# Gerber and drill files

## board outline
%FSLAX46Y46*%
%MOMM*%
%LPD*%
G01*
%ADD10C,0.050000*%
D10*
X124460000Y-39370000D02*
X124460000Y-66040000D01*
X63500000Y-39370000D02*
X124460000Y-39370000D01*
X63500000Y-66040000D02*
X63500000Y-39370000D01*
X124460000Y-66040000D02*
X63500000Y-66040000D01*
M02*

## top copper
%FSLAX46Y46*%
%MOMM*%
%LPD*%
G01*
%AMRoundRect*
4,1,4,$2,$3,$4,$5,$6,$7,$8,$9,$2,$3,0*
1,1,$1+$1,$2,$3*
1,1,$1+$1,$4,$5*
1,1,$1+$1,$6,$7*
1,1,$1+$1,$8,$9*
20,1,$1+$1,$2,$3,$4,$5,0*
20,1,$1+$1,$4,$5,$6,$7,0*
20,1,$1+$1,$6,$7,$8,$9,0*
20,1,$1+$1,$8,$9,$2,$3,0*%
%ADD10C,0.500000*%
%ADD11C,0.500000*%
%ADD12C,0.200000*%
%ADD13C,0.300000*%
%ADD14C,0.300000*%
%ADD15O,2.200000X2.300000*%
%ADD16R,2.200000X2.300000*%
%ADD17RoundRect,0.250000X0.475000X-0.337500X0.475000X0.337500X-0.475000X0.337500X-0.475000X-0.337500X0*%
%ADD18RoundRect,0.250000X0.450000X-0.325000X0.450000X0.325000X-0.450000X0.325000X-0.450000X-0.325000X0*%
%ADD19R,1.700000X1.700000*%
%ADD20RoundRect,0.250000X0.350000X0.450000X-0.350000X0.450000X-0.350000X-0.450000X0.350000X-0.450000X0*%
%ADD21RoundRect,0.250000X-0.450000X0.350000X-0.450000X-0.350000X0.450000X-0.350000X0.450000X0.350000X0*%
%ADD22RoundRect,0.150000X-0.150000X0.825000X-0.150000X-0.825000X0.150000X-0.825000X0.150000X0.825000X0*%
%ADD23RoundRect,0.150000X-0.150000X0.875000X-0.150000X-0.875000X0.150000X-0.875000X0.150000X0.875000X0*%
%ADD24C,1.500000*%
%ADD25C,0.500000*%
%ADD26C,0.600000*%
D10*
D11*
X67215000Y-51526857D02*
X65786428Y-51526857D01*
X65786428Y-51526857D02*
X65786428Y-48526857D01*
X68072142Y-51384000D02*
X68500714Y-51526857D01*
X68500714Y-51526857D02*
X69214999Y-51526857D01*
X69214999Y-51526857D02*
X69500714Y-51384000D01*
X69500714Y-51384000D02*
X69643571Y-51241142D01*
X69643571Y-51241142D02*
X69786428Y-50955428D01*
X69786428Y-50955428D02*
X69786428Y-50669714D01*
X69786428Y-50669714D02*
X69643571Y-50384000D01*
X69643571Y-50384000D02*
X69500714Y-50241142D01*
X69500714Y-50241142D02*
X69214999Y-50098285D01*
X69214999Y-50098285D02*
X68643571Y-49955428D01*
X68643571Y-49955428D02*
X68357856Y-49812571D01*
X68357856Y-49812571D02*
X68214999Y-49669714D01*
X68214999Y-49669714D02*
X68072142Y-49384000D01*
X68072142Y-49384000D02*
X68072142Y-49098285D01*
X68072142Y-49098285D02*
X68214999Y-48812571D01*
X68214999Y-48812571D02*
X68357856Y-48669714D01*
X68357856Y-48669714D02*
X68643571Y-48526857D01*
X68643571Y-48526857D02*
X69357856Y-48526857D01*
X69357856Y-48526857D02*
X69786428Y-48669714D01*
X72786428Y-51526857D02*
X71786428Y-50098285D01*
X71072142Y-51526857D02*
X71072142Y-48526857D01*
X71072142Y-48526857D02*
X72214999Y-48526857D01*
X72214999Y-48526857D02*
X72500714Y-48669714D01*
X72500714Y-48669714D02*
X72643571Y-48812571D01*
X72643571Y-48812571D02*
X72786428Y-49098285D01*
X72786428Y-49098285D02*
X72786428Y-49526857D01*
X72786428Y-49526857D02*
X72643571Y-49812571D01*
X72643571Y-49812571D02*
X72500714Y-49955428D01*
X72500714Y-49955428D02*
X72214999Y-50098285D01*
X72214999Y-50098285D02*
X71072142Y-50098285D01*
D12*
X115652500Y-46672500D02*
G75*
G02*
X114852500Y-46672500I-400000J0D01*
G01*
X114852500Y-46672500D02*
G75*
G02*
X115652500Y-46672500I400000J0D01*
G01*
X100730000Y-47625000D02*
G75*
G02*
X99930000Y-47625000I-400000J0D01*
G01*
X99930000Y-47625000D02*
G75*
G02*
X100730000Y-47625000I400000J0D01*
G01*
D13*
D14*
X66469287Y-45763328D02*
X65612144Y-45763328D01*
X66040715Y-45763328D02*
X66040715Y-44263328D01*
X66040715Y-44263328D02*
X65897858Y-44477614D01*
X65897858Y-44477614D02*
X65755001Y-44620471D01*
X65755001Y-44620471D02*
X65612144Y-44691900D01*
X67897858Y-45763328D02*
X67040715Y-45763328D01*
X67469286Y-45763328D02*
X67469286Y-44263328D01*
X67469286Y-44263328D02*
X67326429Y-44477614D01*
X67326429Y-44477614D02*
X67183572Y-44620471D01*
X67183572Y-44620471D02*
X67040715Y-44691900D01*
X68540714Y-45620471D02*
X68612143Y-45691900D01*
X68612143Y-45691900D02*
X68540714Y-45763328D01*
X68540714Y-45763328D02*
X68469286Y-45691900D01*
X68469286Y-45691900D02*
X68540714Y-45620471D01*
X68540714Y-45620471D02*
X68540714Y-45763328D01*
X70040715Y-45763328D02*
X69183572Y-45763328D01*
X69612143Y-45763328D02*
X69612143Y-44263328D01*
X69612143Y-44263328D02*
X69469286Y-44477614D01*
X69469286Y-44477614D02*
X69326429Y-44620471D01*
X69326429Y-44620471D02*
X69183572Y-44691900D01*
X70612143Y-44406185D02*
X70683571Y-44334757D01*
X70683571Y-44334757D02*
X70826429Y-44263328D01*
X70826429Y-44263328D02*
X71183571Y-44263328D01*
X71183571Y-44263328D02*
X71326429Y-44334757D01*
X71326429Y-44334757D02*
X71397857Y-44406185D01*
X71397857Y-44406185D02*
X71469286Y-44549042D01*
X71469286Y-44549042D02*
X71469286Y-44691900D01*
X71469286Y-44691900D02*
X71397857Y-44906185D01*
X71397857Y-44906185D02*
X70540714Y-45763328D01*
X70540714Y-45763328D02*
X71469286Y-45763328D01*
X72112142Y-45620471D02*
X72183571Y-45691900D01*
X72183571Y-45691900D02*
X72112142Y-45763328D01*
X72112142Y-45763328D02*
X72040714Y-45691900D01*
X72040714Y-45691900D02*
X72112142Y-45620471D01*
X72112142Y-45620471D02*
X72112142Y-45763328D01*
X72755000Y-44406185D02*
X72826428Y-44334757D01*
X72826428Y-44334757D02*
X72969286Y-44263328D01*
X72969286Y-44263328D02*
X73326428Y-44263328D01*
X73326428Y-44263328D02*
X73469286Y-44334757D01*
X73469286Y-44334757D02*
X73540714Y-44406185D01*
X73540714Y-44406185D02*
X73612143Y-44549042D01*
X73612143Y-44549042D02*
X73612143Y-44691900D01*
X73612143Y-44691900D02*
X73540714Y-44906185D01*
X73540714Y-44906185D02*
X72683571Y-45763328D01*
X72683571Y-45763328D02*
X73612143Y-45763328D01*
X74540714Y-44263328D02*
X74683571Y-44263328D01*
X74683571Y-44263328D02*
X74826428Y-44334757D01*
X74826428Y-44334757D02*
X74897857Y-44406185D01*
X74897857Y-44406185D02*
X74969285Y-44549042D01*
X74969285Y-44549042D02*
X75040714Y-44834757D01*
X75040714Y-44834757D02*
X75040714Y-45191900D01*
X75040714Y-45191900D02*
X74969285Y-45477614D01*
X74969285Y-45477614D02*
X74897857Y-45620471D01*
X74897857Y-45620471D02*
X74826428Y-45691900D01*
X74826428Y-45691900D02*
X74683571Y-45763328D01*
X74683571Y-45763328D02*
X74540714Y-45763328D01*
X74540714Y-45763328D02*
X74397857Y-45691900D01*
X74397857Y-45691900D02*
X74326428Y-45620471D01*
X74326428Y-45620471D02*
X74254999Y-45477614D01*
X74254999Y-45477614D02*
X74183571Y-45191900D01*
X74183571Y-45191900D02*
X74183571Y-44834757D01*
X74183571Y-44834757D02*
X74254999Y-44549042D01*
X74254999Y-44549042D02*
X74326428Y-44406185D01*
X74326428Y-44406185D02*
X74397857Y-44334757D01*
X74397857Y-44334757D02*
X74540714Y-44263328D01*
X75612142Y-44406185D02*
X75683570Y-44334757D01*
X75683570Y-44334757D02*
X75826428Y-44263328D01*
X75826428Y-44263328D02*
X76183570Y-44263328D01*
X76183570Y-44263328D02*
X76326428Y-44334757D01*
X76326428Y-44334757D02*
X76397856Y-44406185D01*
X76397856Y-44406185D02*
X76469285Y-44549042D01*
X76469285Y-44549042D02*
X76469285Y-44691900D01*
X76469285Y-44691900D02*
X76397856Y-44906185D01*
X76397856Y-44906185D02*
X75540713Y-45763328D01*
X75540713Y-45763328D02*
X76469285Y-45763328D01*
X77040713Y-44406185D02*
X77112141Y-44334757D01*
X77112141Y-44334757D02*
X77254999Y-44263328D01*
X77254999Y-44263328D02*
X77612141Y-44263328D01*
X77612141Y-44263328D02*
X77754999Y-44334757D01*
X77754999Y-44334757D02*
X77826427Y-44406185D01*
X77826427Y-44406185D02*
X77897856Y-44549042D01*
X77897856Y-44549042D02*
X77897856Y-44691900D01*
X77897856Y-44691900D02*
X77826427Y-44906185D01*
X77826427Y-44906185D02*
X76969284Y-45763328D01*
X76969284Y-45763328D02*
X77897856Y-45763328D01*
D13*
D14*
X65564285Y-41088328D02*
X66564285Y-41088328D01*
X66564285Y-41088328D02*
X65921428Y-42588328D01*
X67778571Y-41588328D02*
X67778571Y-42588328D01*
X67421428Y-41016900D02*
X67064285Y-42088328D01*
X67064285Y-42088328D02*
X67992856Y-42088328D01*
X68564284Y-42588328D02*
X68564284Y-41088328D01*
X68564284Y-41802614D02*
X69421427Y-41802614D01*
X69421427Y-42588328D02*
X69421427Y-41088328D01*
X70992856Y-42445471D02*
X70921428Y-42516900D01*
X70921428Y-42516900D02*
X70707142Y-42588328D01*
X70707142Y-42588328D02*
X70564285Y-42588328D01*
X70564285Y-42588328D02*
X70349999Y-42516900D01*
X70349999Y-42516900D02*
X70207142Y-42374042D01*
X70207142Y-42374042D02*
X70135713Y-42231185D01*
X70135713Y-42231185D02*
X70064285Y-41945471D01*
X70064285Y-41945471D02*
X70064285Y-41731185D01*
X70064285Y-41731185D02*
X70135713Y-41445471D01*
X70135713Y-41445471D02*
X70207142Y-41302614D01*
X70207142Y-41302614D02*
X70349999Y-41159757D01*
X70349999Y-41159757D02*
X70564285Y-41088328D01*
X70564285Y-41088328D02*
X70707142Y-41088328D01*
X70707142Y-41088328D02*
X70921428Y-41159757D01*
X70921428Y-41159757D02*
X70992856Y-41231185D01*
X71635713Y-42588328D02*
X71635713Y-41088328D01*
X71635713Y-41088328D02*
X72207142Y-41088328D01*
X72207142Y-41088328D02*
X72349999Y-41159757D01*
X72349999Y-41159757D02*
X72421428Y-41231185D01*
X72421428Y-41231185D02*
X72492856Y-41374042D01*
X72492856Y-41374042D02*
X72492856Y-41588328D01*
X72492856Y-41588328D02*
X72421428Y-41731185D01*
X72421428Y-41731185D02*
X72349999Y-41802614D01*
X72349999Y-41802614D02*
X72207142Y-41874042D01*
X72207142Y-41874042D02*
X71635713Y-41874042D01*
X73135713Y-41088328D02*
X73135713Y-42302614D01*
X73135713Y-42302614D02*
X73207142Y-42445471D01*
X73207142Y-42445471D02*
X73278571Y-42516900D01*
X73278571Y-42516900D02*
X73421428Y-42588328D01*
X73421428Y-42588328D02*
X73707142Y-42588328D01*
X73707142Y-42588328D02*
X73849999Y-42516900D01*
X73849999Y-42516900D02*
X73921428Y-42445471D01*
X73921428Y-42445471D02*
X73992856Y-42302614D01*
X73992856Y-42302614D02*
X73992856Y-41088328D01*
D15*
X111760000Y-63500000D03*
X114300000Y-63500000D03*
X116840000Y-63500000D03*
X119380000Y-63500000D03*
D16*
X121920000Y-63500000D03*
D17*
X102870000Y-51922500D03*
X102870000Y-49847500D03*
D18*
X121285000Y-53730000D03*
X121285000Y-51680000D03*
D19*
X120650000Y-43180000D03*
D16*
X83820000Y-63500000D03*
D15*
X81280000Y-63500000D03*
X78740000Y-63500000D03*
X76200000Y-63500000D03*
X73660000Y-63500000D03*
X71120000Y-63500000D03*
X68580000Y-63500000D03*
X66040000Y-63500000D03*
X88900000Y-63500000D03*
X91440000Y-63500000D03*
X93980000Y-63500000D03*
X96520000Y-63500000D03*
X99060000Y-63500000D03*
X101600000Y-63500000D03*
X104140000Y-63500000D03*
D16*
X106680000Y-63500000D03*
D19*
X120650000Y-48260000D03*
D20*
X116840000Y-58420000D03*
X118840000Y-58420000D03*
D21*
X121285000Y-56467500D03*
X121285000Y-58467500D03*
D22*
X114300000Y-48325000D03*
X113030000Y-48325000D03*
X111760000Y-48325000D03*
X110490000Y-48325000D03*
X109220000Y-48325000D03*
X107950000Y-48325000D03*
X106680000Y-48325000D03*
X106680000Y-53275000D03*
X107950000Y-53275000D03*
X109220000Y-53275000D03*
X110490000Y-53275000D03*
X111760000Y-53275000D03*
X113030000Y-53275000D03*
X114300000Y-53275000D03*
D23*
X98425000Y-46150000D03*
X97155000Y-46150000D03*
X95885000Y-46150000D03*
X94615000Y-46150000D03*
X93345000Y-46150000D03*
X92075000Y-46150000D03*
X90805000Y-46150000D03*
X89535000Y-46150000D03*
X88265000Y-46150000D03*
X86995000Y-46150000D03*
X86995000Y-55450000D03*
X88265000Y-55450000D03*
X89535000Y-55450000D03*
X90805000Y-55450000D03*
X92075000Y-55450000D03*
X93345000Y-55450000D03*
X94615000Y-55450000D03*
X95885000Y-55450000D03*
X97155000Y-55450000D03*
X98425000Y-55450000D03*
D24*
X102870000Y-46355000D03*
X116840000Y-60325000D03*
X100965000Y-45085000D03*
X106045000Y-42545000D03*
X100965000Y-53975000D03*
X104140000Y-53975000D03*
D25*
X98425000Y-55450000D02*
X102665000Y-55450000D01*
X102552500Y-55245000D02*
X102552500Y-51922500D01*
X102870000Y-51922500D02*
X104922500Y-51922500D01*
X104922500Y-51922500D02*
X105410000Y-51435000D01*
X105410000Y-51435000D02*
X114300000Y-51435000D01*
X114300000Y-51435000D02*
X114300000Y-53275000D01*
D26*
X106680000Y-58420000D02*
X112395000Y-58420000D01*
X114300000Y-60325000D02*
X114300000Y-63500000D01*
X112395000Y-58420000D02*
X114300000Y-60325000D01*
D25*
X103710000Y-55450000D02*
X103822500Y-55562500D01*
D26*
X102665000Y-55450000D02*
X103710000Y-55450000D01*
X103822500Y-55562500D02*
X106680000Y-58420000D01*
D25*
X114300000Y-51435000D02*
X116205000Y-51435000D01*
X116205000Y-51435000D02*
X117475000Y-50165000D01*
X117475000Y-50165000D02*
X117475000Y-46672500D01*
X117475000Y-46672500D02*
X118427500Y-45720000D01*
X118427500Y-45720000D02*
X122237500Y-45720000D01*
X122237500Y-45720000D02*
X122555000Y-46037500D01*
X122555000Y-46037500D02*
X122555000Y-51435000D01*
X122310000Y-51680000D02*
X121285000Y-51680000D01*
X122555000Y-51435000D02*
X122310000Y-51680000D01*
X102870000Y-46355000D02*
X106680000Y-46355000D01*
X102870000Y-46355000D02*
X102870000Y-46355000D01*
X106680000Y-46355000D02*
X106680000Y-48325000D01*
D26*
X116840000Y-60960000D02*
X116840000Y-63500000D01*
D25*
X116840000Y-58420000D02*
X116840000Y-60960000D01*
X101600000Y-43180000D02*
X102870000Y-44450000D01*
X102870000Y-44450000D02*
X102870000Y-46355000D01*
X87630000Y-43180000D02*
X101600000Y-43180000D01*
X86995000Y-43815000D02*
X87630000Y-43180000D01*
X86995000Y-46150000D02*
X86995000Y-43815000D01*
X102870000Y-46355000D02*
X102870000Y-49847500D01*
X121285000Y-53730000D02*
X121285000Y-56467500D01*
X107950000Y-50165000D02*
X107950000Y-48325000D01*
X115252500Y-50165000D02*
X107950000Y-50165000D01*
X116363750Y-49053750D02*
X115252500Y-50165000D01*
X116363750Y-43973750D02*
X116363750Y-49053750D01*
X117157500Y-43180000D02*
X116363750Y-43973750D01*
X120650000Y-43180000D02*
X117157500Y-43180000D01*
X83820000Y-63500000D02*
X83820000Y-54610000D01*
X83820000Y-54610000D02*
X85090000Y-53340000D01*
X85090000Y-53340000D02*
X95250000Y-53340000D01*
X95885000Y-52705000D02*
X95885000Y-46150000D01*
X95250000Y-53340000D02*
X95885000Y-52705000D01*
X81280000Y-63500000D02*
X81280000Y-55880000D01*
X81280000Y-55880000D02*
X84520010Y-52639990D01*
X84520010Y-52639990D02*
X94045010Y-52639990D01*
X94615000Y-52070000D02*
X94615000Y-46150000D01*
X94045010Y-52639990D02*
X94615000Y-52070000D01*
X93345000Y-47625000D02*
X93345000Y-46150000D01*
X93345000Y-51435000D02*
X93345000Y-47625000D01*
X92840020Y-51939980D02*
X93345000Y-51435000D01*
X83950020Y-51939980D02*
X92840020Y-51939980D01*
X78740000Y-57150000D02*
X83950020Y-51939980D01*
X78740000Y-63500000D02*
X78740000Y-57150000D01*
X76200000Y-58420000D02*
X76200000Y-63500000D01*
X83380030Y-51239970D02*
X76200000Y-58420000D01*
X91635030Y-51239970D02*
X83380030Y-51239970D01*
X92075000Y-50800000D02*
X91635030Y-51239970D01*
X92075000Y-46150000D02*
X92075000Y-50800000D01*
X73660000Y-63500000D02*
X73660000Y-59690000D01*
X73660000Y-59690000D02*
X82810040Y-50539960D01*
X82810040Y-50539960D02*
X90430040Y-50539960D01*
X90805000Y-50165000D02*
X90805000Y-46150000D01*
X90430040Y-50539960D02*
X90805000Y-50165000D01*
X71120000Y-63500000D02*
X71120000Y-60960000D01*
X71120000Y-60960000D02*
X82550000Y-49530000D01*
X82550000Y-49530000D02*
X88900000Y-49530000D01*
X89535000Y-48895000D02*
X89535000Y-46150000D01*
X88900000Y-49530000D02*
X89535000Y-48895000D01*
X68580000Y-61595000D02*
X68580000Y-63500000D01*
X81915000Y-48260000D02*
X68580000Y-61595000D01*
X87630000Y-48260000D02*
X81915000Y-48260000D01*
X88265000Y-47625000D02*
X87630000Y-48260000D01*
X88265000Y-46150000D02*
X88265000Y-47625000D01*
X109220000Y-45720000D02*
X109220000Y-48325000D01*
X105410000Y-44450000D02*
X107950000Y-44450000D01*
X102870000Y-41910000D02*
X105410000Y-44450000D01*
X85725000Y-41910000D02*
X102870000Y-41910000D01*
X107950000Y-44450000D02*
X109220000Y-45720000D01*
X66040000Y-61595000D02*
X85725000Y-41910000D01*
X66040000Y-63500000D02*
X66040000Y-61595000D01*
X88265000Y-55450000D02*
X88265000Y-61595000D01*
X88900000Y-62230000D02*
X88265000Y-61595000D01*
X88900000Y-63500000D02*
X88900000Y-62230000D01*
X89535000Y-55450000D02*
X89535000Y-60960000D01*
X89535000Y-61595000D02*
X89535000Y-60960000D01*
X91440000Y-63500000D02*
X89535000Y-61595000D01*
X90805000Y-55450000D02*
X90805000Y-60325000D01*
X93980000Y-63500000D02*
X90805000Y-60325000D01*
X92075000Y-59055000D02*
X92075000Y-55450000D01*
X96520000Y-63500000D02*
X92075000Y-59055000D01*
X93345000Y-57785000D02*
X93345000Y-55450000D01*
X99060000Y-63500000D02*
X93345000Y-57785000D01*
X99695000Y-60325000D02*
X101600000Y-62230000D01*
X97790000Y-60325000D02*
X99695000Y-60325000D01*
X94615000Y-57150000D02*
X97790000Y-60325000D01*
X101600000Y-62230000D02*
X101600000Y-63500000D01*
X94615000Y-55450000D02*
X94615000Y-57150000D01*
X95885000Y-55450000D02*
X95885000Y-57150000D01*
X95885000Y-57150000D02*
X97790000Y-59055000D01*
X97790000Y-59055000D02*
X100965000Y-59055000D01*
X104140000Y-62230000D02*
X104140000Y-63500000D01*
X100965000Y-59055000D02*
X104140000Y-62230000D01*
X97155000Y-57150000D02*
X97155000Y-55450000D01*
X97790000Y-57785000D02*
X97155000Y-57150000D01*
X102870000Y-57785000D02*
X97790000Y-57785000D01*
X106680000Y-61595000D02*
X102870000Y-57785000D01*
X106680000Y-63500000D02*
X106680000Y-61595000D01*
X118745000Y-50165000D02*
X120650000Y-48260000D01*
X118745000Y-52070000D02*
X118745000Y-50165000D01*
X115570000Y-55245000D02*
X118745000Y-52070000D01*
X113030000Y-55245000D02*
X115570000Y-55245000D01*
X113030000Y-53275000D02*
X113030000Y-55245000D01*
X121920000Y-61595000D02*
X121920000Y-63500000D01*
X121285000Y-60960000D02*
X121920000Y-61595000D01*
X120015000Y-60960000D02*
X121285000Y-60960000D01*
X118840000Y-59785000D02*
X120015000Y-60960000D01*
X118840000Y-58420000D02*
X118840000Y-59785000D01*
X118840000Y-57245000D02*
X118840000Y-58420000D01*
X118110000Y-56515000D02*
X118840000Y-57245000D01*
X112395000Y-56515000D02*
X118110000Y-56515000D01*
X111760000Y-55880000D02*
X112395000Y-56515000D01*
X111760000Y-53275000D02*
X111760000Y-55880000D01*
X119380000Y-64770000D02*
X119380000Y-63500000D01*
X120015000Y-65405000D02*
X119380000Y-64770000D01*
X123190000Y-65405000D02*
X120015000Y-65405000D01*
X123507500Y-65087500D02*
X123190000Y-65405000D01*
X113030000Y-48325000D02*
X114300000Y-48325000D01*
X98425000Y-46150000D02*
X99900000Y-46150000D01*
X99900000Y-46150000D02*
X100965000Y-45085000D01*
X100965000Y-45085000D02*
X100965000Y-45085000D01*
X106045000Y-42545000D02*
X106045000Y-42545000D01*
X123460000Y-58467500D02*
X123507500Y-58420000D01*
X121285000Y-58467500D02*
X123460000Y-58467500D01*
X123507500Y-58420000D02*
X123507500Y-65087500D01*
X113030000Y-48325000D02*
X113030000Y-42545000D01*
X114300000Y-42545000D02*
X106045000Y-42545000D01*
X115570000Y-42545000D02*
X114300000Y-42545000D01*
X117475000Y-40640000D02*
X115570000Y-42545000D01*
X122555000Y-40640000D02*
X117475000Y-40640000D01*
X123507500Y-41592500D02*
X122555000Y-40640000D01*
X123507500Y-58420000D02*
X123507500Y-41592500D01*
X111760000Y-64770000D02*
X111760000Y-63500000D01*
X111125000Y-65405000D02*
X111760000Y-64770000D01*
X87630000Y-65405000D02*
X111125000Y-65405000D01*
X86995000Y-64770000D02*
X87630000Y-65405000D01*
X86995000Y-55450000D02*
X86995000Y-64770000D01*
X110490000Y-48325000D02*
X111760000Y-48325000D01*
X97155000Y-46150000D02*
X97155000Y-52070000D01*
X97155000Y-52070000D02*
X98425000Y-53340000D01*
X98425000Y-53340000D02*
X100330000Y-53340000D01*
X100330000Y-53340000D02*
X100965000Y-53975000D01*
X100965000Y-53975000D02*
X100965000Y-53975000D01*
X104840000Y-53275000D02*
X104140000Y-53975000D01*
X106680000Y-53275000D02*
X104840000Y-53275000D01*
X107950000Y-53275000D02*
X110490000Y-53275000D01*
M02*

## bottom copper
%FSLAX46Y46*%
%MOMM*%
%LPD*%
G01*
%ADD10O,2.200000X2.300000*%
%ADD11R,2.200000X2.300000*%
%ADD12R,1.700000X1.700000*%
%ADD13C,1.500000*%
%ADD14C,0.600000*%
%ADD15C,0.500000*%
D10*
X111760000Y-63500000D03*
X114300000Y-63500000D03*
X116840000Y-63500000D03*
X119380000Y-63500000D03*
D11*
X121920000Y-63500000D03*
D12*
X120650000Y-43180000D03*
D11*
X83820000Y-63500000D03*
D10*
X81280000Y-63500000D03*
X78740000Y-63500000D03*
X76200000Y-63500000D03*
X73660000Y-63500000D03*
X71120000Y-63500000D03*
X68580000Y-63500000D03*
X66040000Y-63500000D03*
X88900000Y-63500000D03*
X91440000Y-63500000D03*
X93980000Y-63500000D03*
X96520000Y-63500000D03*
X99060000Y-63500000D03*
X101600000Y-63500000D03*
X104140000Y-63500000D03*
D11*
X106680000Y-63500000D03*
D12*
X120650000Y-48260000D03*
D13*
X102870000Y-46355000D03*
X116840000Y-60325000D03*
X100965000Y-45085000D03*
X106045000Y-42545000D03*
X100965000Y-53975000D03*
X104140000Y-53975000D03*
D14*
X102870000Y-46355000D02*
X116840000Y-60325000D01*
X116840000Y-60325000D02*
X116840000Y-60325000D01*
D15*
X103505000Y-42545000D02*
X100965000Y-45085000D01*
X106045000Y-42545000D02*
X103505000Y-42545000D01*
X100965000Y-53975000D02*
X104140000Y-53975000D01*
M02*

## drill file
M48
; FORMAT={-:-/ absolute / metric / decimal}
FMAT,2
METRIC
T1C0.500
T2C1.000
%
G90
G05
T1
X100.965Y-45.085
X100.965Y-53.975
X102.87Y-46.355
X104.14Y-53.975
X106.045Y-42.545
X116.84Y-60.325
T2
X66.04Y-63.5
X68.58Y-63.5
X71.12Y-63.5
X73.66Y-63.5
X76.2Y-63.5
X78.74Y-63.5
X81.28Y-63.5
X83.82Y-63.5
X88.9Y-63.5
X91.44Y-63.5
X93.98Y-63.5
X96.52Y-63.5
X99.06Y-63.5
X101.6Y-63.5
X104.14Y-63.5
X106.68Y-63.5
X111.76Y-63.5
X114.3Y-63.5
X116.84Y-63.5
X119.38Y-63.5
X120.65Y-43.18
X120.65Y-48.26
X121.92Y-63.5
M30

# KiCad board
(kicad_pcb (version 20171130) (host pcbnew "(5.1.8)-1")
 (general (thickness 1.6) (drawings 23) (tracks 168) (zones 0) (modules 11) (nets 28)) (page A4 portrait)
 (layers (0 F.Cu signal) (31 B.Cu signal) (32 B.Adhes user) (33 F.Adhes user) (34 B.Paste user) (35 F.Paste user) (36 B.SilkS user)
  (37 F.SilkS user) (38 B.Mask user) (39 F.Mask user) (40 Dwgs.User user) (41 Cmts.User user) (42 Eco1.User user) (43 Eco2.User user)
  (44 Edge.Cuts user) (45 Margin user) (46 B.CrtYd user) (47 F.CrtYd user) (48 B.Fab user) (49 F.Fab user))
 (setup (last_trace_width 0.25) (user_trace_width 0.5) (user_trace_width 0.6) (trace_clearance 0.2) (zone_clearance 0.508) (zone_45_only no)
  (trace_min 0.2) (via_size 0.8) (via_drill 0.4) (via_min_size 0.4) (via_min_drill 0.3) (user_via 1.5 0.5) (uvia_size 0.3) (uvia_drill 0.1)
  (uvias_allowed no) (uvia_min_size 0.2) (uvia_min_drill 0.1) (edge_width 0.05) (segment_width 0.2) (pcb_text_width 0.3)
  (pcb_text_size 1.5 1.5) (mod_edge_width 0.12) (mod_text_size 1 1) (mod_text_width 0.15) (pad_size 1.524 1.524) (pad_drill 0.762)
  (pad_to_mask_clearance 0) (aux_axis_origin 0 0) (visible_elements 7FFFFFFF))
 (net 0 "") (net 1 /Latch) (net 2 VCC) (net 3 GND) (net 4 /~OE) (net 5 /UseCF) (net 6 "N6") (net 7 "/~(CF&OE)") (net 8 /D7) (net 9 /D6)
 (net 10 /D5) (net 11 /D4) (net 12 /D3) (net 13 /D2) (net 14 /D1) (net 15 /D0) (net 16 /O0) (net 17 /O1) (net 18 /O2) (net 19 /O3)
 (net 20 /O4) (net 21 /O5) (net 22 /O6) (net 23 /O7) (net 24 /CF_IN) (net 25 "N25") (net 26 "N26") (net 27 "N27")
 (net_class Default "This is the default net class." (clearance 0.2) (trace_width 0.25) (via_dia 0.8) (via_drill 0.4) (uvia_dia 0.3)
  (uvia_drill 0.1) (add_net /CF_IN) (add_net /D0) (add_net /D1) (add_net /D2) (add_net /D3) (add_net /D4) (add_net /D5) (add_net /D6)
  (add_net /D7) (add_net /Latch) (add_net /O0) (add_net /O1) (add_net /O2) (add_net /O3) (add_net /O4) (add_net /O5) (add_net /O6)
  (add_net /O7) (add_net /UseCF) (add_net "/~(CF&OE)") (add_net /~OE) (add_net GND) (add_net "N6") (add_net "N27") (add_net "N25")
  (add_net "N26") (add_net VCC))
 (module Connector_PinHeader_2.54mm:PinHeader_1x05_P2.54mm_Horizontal (layer F.Cu) (at 121.92 63.5 270)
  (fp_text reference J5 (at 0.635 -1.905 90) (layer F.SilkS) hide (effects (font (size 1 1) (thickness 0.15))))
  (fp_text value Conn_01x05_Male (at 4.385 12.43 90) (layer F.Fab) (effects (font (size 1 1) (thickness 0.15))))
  (pad 5 thru_hole oval (at 0 10.16 270) (size 2.3 2.2) (drill 1) (layers *.Cu *.Mask) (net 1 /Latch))
  (pad 4 thru_hole oval (at 0 7.62 270) (size 2.3 2.2) (drill 1) (layers *.Cu *.Mask) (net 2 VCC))
  (pad 3 thru_hole oval (at 0 5.08 270) (size 2.3 2.2) (drill 1) (layers *.Cu *.Mask) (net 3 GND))
  (pad 2 thru_hole oval (at 0 2.54 270) (size 2.3 2.2) (drill 1) (layers *.Cu *.Mask) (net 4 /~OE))
  (pad 1 thru_hole rect (at 0 0 270) (size 2.3 2.2) (drill 1) (layers *.Cu *.Mask) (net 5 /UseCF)))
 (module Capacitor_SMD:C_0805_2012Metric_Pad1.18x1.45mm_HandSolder (layer F.Cu) (at 102.87 50.885 90)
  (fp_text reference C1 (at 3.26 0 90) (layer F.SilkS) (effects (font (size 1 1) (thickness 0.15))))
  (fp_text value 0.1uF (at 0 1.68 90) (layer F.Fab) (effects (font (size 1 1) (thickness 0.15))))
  (pad 1 smd roundrect (at -1.0375 0 90) (size 1.175 1.45) (layers F.Cu F.Paste F.Mask) (roundrect_rratio 0.212766) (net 2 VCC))
  (pad 2 smd roundrect (at 1.0375 0 90) (size 1.175 1.45) (layers F.Cu F.Paste F.Mask) (roundrect_rratio 0.212766) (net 3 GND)))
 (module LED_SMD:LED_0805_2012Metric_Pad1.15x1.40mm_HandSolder (layer F.Cu) (at 121.285 52.705 90)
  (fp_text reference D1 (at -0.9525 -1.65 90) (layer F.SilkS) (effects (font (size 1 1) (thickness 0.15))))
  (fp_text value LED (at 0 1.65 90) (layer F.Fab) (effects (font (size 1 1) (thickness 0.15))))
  (pad 1 smd roundrect (at -1.025 0 90) (size 1.15 1.4) (layers F.Cu F.Paste F.Mask) (roundrect_rratio 0.217391) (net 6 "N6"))
  (pad 2 smd roundrect (at 1.025 0 90) (size 1.15 1.4) (layers F.Cu F.Paste F.Mask) (roundrect_rratio 0.217391) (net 2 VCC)))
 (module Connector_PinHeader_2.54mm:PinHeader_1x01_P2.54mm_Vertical (layer F.Cu) (at 120.65 43.18)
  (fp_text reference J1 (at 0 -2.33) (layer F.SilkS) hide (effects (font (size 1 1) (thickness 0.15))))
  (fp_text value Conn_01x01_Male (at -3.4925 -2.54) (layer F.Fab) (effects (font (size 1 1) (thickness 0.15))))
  (pad 1 thru_hole rect (at 0 0) (size 1.7 1.7) (drill 1) (layers *.Cu *.Mask) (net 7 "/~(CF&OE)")))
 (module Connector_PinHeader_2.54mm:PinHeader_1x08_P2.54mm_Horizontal (layer F.Cu) (at 83.82 63.5 270)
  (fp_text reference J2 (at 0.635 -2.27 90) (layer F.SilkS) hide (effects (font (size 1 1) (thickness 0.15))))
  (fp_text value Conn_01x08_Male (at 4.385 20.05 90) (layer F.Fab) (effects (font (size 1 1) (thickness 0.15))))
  (pad 1 thru_hole rect (at 0 0 270) (size 2.3 2.2) (drill 1) (layers *.Cu *.Mask) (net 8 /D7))
  (pad 2 thru_hole oval (at 0 2.54 270) (size 2.3 2.2) (drill 1) (layers *.Cu *.Mask) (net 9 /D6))
  (pad 3 thru_hole oval (at 0 5.08 270) (size 2.3 2.2) (drill 1) (layers *.Cu *.Mask) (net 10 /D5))
  (pad 4 thru_hole oval (at 0 7.62 270) (size 2.3 2.2) (drill 1) (layers *.Cu *.Mask) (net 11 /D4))
  (pad 5 thru_hole oval (at 0 10.16 270) (size 2.3 2.2) (drill 1) (layers *.Cu *.Mask) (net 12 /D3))
  (pad 6 thru_hole oval (at 0 12.7 270) (size 2.3 2.2) (drill 1) (layers *.Cu *.Mask) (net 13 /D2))
  (pad 7 thru_hole oval (at 0 15.24 270) (size 2.3 2.2) (drill 1) (layers *.Cu *.Mask) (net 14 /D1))
  (pad 8 thru_hole oval (at 0 17.78 270) (size 2.3 2.2) (drill 1) (layers *.Cu *.Mask) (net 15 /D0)))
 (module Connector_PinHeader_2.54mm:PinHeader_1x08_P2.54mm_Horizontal (layer F.Cu) (at 106.68 63.5 270)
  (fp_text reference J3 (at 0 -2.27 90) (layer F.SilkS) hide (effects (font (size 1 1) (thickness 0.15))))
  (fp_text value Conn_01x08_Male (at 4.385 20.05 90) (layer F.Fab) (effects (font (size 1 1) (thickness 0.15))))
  (pad 8 thru_hole oval (at 0 17.78 270) (size 2.3 2.2) (drill 1) (layers *.Cu *.Mask) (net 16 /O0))
  (pad 7 thru_hole oval (at 0 15.24 270) (size 2.3 2.2) (drill 1) (layers *.Cu *.Mask) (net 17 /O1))
  (pad 6 thru_hole oval (at 0 12.7 270) (size 2.3 2.2) (drill 1) (layers *.Cu *.Mask) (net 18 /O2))
  (pad 5 thru_hole oval (at 0 10.16 270) (size 2.3 2.2) (drill 1) (layers *.Cu *.Mask) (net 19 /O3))
  (pad 4 thru_hole oval (at 0 7.62 270) (size 2.3 2.2) (drill 1) (layers *.Cu *.Mask) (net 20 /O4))
  (pad 3 thru_hole oval (at 0 5.08 270) (size 2.3 2.2) (drill 1) (layers *.Cu *.Mask) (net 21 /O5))
  (pad 2 thru_hole oval (at 0 2.54 270) (size 2.3 2.2) (drill 1) (layers *.Cu *.Mask) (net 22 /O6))
  (pad 1 thru_hole rect (at 0 0 270) (size 2.3 2.2) (drill 1) (layers *.Cu *.Mask) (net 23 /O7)))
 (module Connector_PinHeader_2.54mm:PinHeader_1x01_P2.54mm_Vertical (layer F.Cu) (at 120.65 48.26)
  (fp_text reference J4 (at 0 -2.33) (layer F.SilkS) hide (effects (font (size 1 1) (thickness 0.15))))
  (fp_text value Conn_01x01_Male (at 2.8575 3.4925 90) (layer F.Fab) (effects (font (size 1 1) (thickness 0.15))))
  (pad 1 thru_hole rect (at 0 0) (size 1.7 1.7) (drill 1) (layers *.Cu *.Mask) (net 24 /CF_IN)))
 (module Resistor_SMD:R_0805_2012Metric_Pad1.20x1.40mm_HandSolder (layer F.Cu) (at 117.84 58.42 180)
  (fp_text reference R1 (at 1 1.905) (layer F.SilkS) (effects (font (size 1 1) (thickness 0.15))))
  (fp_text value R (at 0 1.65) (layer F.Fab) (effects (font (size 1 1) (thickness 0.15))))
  (pad 2 smd roundrect (at 1 0 180) (size 1.2 1.4) (layers F.Cu F.Paste F.Mask) (roundrect_rratio 0.208333) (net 3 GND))
  (pad 1 smd roundrect (at -1 0 180) (size 1.2 1.4) (layers F.Cu F.Paste F.Mask) (roundrect_rratio 0.208333) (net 5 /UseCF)))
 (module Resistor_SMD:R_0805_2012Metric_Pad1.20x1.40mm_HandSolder (layer F.Cu) (at 121.285 57.4675 270)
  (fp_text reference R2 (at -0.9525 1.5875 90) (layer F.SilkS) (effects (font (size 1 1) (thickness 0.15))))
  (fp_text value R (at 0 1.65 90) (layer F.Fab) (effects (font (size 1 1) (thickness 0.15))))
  (pad 1 smd roundrect (at -1 0 270) (size 1.2 1.4) (layers F.Cu F.Paste F.Mask) (roundrect_rratio 0.208333) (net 6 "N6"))
  (pad 2 smd roundrect (at 1 0 270) (size 1.2 1.4) (layers F.Cu F.Paste F.Mask) (roundrect_rratio 0.208333) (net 4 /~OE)))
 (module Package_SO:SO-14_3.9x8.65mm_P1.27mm (layer F.Cu) (at 110.49 50.8 270)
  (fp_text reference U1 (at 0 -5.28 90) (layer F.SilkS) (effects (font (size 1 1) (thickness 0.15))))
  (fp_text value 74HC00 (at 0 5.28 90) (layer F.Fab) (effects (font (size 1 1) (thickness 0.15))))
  (pad 1 smd roundrect (at -2.475 -3.81 270) (size 1.95 0.6) (layers F.Cu F.Paste F.Mask) (roundrect_rratio 0.25) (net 4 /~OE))
  (pad 2 smd roundrect (at -2.475 -2.54 270) (size 1.95 0.6) (layers F.Cu F.Paste F.Mask) (roundrect_rratio 0.25) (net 4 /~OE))
  (pad 3 smd roundrect (at -2.475 -1.27 270) (size 1.95 0.6) (layers F.Cu F.Paste F.Mask) (roundrect_rratio 0.25) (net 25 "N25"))
  (pad 4 smd roundrect (at -2.475 0 270) (size 1.95 0.6) (layers F.Cu F.Paste F.Mask) (roundrect_rratio 0.25) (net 25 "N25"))
  (pad 5 smd roundrect (at -2.475 1.27 270) (size 1.95 0.6) (layers F.Cu F.Paste F.Mask) (roundrect_rratio 0.25) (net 15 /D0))
  (pad 6 smd roundrect (at -2.475 2.54 270) (size 1.95 0.6) (layers F.Cu F.Paste F.Mask) (roundrect_rratio 0.25) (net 7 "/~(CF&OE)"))
  (pad 7 smd roundrect (at -2.475 3.81 270) (size 1.95 0.6) (layers F.Cu F.Paste F.Mask) (roundrect_rratio 0.25) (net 3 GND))
  (pad 8 smd roundrect (at 2.475 3.81 270) (size 1.95 0.6) (layers F.Cu F.Paste F.Mask) (roundrect_rratio 0.25) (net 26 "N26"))
  (pad 9 smd roundrect (at 2.475 2.54 270) (size 1.95 0.6) (layers F.Cu F.Paste F.Mask) (roundrect_rratio 0.25) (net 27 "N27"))
  (pad 10 smd roundrect (at 2.475 1.27 270) (size 1.95 0.6) (layers F.Cu F.Paste F.Mask) (roundrect_rratio 0.25) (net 27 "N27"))
  (pad 11 smd roundrect (at 2.475 0 270) (size 1.95 0.6) (layers F.Cu F.Paste F.Mask) (roundrect_rratio 0.25) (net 27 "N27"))
  (pad 12 smd roundrect (at 2.475 -1.27 270) (size 1.95 0.6) (layers F.Cu F.Paste F.Mask) (roundrect_rratio 0.25) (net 5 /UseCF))
  (pad 13 smd roundrect (at 2.475 -2.54 270) (size 1.95 0.6) (layers F.Cu F.Paste F.Mask) (roundrect_rratio 0.25) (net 24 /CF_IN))
  (pad 14 smd roundrect (at 2.475 -3.81 270) (size 1.95 0.6) (layers F.Cu F.Paste F.Mask) (roundrect_rratio 0.25) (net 2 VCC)))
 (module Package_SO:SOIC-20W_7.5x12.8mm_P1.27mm (layer F.Cu) (at 92.71 50.8 270)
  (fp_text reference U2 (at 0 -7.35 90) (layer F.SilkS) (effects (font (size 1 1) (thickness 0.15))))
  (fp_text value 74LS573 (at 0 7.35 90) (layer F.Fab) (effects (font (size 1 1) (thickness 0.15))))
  (pad 1 smd roundrect (at -4.65 -5.715 270) (size 2.05 0.6) (layers F.Cu F.Paste F.Mask) (roundrect_rratio 0.25) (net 4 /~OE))
  (pad 2 smd roundrect (at -4.65 -4.445 270) (size 2.05 0.6) (layers F.Cu F.Paste F.Mask) (roundrect_rratio 0.25) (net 26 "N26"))
  (pad 3 smd roundrect (at -4.65 -3.175 270) (size 2.05 0.6) (layers F.Cu F.Paste F.Mask) (roundrect_rratio 0.25) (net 8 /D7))
  (pad 4 smd roundrect (at -4.65 -1.905 270) (size 2.05 0.6) (layers F.Cu F.Paste F.Mask) (roundrect_rratio 0.25) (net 9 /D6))
  (pad 5 smd roundrect (at -4.65 -0.635 270) (size 2.05 0.6) (layers F.Cu F.Paste F.Mask) (roundrect_rratio 0.25) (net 10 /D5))
  (pad 6 smd roundrect (at -4.65 0.635 270) (size 2.05 0.6) (layers F.Cu F.Paste F.Mask) (roundrect_rratio 0.25) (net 11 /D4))
  (pad 7 smd roundrect (at -4.65 1.905 270) (size 2.05 0.6) (layers F.Cu F.Paste F.Mask) (roundrect_rratio 0.25) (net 12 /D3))
  (pad 8 smd roundrect (at -4.65 3.175 270) (size 2.05 0.6) (layers F.Cu F.Paste F.Mask) (roundrect_rratio 0.25) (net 13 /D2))
  (pad 9 smd roundrect (at -4.65 4.445 270) (size 2.05 0.6) (layers F.Cu F.Paste F.Mask) (roundrect_rratio 0.25) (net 14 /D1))
  (pad 10 smd roundrect (at -4.65 5.715 270) (size 2.05 0.6) (layers F.Cu F.Paste F.Mask) (roundrect_rratio 0.25) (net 3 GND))
  (pad 11 smd roundrect (at 4.65 5.715 270) (size 2.05 0.6) (layers F.Cu F.Paste F.Mask) (roundrect_rratio 0.25) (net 1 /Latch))
  (pad 12 smd roundrect (at 4.65 4.445 270) (size 2.05 0.6) (layers F.Cu F.Paste F.Mask) (roundrect_rratio 0.25) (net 16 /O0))
  (pad 13 smd roundrect (at 4.65 3.175 270) (size 2.05 0.6) (layers F.Cu F.Paste F.Mask) (roundrect_rratio 0.25) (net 17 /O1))
  (pad 14 smd roundrect (at 4.65 1.905 270) (size 2.05 0.6) (layers F.Cu F.Paste F.Mask) (roundrect_rratio 0.25) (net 18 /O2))
  (pad 15 smd roundrect (at 4.65 0.635 270) (size 2.05 0.6) (layers F.Cu F.Paste F.Mask) (roundrect_rratio 0.25) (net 19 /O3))
  (pad 16 smd roundrect (at 4.65 -0.635 270) (size 2.05 0.6) (layers F.Cu F.Paste F.Mask) (roundrect_rratio 0.25) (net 20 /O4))
  (pad 17 smd roundrect (at 4.65 -1.905 270) (size 2.05 0.6) (layers F.Cu F.Paste F.Mask) (roundrect_rratio 0.25) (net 21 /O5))
  (pad 18 smd roundrect (at 4.65 -3.175 270) (size 2.05 0.6) (layers F.Cu F.Paste F.Mask) (roundrect_rratio 0.25) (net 22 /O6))
  (pad 19 smd roundrect (at 4.65 -4.445 270) (size 2.05 0.6) (layers F.Cu F.Paste F.Mask) (roundrect_rratio 0.25) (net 23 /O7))
  (pad 20 smd roundrect (at 4.65 -5.715 270) (size 2.05 0.6) (layers F.Cu F.Paste F.Mask) (roundrect_rratio 0.25) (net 2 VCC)))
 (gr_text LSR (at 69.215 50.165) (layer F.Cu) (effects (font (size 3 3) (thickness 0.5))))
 (gr_circle (center 115.2525 46.6725) (end 115.6525 46.6725) (layer F.Cu) (width 0.2))
 (gr_circle (center 100.33 47.625) (end 100.73 47.625) (layer F.Cu) (width 0.2))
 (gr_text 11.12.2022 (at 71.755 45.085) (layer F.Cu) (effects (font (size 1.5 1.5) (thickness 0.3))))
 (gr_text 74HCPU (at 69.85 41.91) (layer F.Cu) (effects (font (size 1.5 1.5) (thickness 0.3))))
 (gr_line (start 124.46 39.37) (end 124.46 66.04) (layer Edge.Cuts) (width 0.05))
 (gr_line (start 63.5 39.37) (end 124.46 39.37) (layer Edge.Cuts) (width 0.05))
 (gr_line (start 63.5 66.04) (end 63.5 39.37) (layer Edge.Cuts) (width 0.05))
 (gr_line (start 124.46 66.04) (end 63.5 66.04) (layer Edge.Cuts) (width 0.05))
 (segment (start 98.425 55.45) (end 102.665 55.45) (width 0.5) (layer F.Cu) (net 2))
 (segment (start 102.5525 55.245) (end 102.5525 51.9225) (width 0.5) (layer F.Cu) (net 2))
 (segment (start 102.87 51.9225) (end 104.9225 51.9225) (width 0.5) (layer F.Cu) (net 2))
 (segment (start 104.9225 51.9225) (end 105.41 51.435) (width 0.5) (layer F.Cu) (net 2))
 (segment (start 105.41 51.435) (end 114.3 51.435) (width 0.5) (layer F.Cu) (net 2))
 (segment (start 114.3 51.435) (end 114.3 53.275) (width 0.5) (layer F.Cu) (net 2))
 (segment (start 106.68 58.42) (end 112.395 58.42) (width 0.6) (layer F.Cu) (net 2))
 (segment (start 114.3 60.325) (end 114.3 63.5) (width 0.6) (layer F.Cu) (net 2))
 (segment (start 112.395 58.42) (end 114.3 60.325) (width 0.6) (layer F.Cu) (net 2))
 (segment (start 103.71 55.45) (end 103.8225 55.5625) (width 0.5) (layer F.Cu) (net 2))
 (segment (start 102.665 55.45) (end 103.71 55.45) (width 0.6) (layer F.Cu) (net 2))
 (segment (start 103.8225 55.5625) (end 106.68 58.42) (width 0.6) (layer F.Cu) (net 2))
 (segment (start 114.3 51.435) (end 116.205 51.435) (width 0.5) (layer F.Cu) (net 2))
 (segment (start 116.205 51.435) (end 117.475 50.165) (width 0.5) (layer F.Cu) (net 2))
 (segment (start 117.475 50.165) (end 117.475 46.6725) (width 0.5) (layer F.Cu) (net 2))
 (segment (start 117.475 46.6725) (end 118.4275 45.72) (width 0.5) (layer F.Cu) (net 2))
 (segment (start 118.4275 45.72) (end 122.2375 45.72) (width 0.5) (layer F.Cu) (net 2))
 (segment (start 122.2375 45.72) (end 122.555 46.0375) (width 0.5) (layer F.Cu) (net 2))
 (segment (start 122.555 46.0375) (end 122.555 51.435) (width 0.5) (layer F.Cu) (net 2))
 (segment (start 122.31 51.68) (end 121.285 51.68) (width 0.5) (layer F.Cu) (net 2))
 (segment (start 122.555 51.435) (end 122.31 51.68) (width 0.5) (layer F.Cu) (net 2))
 (segment (start 102.87 46.355) (end 106.68 46.355) (width 0.5) (layer F.Cu) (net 3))
 (segment (start 102.87 46.355) (end 102.87 46.355) (width 0.5) (layer F.Cu) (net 3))
 (segment (start 106.68 46.355) (end 106.68 48.325) (width 0.5) (layer F.Cu) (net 3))
 (segment (start 116.84 60.96) (end 116.84 63.5) (width 0.6) (layer F.Cu) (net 3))
 (segment (start 116.84 58.42) (end 116.84 60.96) (width 0.5) (layer F.Cu) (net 3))
 (segment (start 101.6 43.18) (end 102.87 44.45) (width 0.5) (layer F.Cu) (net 3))
 (segment (start 102.87 44.45) (end 102.87 46.355) (width 0.5) (layer F.Cu) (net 3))
 (segment (start 87.63 43.18) (end 101.6 43.18) (width 0.5) (layer F.Cu) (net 3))
 (segment (start 86.995 43.815) (end 87.63 43.18) (width 0.5) (layer F.Cu) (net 3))
 (segment (start 86.995 46.15) (end 86.995 43.815) (width 0.5) (layer F.Cu) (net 3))
 (segment (start 102.87 46.355) (end 102.87 49.8475) (width 0.5) (layer F.Cu) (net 3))
 (via (at 102.87 46.355) (size 1.5) (drill 0.5) (layers F.Cu B.Cu) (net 3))
 (segment (start 102.87 46.355) (end 116.84 60.325) (width 0.6) (layer B.Cu) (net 3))
 (segment (start 116.84 60.325) (end 116.84 60.325) (width 0.6) (layer B.Cu) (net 3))
 (via (at 116.84 60.325) (size 1.5) (drill 0.5) (layers F.Cu B.Cu) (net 3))
 (segment (start 121.285 53.73) (end 121.285 56.4675) (width 0.5) (layer F.Cu) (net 6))
 (segment (start 107.95 50.165) (end 107.95 48.325) (width 0.5) (layer F.Cu) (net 7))
 (segment (start 115.2525 50.165) (end 107.95 50.165) (width 0.5) (layer F.Cu) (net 7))
 (segment (start 116.36375 49.05375) (end 115.2525 50.165) (width 0.5) (layer F.Cu) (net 7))
 (segment (start 116.36375 43.97375) (end 116.36375 49.05375) (width 0.5) (layer F.Cu) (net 7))
 (segment (start 117.1575 43.18) (end 116.36375 43.97375) (width 0.5) (layer F.Cu) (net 7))
 (segment (start 120.65 43.18) (end 117.1575 43.18) (width 0.5) (layer F.Cu) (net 7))
 (segment (start 83.82 63.5) (end 83.82 54.61) (width 0.5) (layer F.Cu) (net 8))
 (segment (start 83.82 54.61) (end 85.09 53.34) (width 0.5) (layer F.Cu) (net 8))
 (segment (start 85.09 53.34) (end 95.25 53.34) (width 0.5) (layer F.Cu) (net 8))
 (segment (start 95.885 52.705) (end 95.885 46.15) (width 0.5) (layer F.Cu) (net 8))
 (segment (start 95.25 53.34) (end 95.885 52.705) (width 0.5) (layer F.Cu) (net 8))
 (segment (start 81.28 63.5) (end 81.28 55.88) (width 0.5) (layer F.Cu) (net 9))
 (segment (start 81.28 55.88) (end 84.52001 52.63999) (width 0.5) (layer F.Cu) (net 9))
 (segment (start 84.52001 52.63999) (end 94.04501 52.63999) (width 0.5) (layer F.Cu) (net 9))
 (segment (start 94.615 52.07) (end 94.615 46.15) (width 0.5) (layer F.Cu) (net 9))
 (segment (start 94.04501 52.63999) (end 94.615 52.07) (width 0.5) (layer F.Cu) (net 9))
 (segment (start 93.345 47.625) (end 93.345 46.15) (width 0.5) (layer F.Cu) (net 10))
 (segment (start 93.345 51.435) (end 93.345 47.625) (width 0.5) (layer F.Cu) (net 10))
 (segment (start 92.84002 51.93998) (end 93.345 51.435) (width 0.5) (layer F.Cu) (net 10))
 (segment (start 83.95002 51.93998) (end 92.84002 51.93998) (width 0.5) (layer F.Cu) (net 10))
 (segment (start 78.74 57.15) (end 83.95002 51.93998) (width 0.5) (layer F.Cu) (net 10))
 (segment (start 78.74 63.5) (end 78.74 57.15) (width 0.5) (layer F.Cu) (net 10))
 (segment (start 76.2 58.42) (end 76.2 63.5) (width 0.5) (layer F.Cu) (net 11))
 (segment (start 83.38003 51.23997) (end 76.2 58.42) (width 0.5) (layer F.Cu) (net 11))
 (segment (start 91.63503 51.23997) (end 83.38003 51.23997) (width 0.5) (layer F.Cu) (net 11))
 (segment (start 92.075 50.8) (end 91.63503 51.23997) (width 0.5) (layer F.Cu) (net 11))
 (segment (start 92.075 46.15) (end 92.075 50.8) (width 0.5) (layer F.Cu) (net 11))
 (segment (start 73.66 63.5) (end 73.66 59.69) (width 0.5) (layer F.Cu) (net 12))
 (segment (start 73.66 59.69) (end 82.81004 50.53996) (width 0.5) (layer F.Cu) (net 12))
 (segment (start 82.81004 50.53996) (end 90.43004 50.53996) (width 0.5) (layer F.Cu) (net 12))
 (segment (start 90.805 50.165) (end 90.805 46.15) (width 0.5) (layer F.Cu) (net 12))
 (segment (start 90.43004 50.53996) (end 90.805 50.165) (width 0.5) (layer F.Cu) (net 12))
 (segment (start 71.12 63.5) (end 71.12 60.96) (width 0.5) (layer F.Cu) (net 13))
 (segment (start 71.12 60.96) (end 82.55 49.53) (width 0.5) (layer F.Cu) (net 13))
 (segment (start 82.55 49.53) (end 88.9 49.53) (width 0.5) (layer F.Cu) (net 13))
 (segment (start 89.535 48.895) (end 89.535 46.15) (width 0.5) (layer F.Cu) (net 13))
 (segment (start 88.9 49.53) (end 89.535 48.895) (width 0.5) (layer F.Cu) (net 13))
 (segment (start 68.58 61.595) (end 68.58 63.5) (width 0.5) (layer F.Cu) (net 14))
 (segment (start 81.915 48.26) (end 68.58 61.595) (width 0.5) (layer F.Cu) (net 14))
 (segment (start 87.63 48.26) (end 81.915 48.26) (width 0.5) (layer F.Cu) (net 14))
 (segment (start 88.265 47.625) (end 87.63 48.26) (width 0.5) (layer F.Cu) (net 14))
 (segment (start 88.265 46.15) (end 88.265 47.625) (width 0.5) (layer F.Cu) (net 14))
 (segment (start 109.22 45.72) (end 109.22 48.325) (width 0.5) (layer F.Cu) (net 15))
 (segment (start 105.41 44.45) (end 107.95 44.45) (width 0.5) (layer F.Cu) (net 15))
 (segment (start 102.87 41.91) (end 105.41 44.45) (width 0.5) (layer F.Cu) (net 15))
 (segment (start 85.725 41.91) (end 102.87 41.91) (width 0.5) (layer F.Cu) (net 15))
 (segment (start 107.95 44.45) (end 109.22 45.72) (width 0.5) (layer F.Cu) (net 15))
 (segment (start 66.04 61.595) (end 85.725 41.91) (width 0.5) (layer F.Cu) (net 15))
 (segment (start 66.04 63.5) (end 66.04 61.595) (width 0.5) (layer F.Cu) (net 15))
 (segment (start 88.265 55.45) (end 88.265 61.595) (width 0.5) (layer F.Cu) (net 16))
 (segment (start 88.9 62.23) (end 88.265 61.595) (width 0.5) (layer F.Cu) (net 16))
 (segment (start 88.9 63.5) (end 88.9 62.23) (width 0.5) (layer F.Cu) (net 16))
 (segment (start 89.535 55.45) (end 89.535 60.96) (width 0.5) (layer F.Cu) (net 17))
 (segment (start 89.535 61.595) (end 89.535 60.96) (width 0.5) (layer F.Cu) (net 17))
 (segment (start 91.44 63.5) (end 89.535 61.595) (width 0.5) (layer F.Cu) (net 17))
 (segment (start 90.805 55.45) (end 90.805 60.325) (width 0.5) (layer F.Cu) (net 18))
 (segment (start 93.98 63.5) (end 90.805 60.325) (width 0.5) (layer F.Cu) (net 18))
 (segment (start 92.075 59.055) (end 92.075 55.45) (width 0.5) (layer F.Cu) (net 19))
 (segment (start 96.52 63.5) (end 92.075 59.055) (width 0.5) (layer F.Cu) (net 19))
 (segment (start 93.345 57.785) (end 93.345 55.45) (width 0.5) (layer F.Cu) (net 20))
 (segment (start 99.06 63.5) (end 93.345 57.785) (width 0.5) (layer F.Cu) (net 20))
 (segment (start 99.695 60.325) (end 101.6 62.23) (width 0.5) (layer F.Cu) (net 21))
 (segment (start 97.79 60.325) (end 99.695 60.325) (width 0.5) (layer F.Cu) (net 21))
 (segment (start 94.615 57.15) (end 97.79 60.325) (width 0.5) (layer F.Cu) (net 21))
 (segment (start 101.6 62.23) (end 101.6 63.5) (width 0.5) (layer F.Cu) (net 21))
 (segment (start 94.615 55.45) (end 94.615 57.15) (width 0.5) (layer F.Cu) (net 21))
 (segment (start 95.885 55.45) (end 95.885 57.15) (width 0.5) (layer F.Cu) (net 22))
 (segment (start 95.885 57.15) (end 97.79 59.055) (width 0.5) (layer F.Cu) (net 22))
 (segment (start 97.79 59.055) (end 100.965 59.055) (width 0.5) (layer F.Cu) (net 22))
 (segment (start 104.14 62.23) (end 104.14 63.5) (width 0.5) (layer F.Cu) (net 22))
 (segment (start 100.965 59.055) (end 104.14 62.23) (width 0.5) (layer F.Cu) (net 22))
 (segment (start 97.155 57.15) (end 97.155 55.45) (width 0.5) (layer F.Cu) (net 23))
 (segment (start 97.79 57.785) (end 97.155 57.15) (width 0.5) (layer F.Cu) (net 23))
 (segment (start 102.87 57.785) (end 97.79 57.785) (width 0.5) (layer F.Cu) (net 23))
 (segment (start 106.68 61.595) (end 102.87 57.785) (width 0.5) (layer F.Cu) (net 23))
 (segment (start 106.68 63.5) (end 106.68 61.595) (width 0.5) (layer F.Cu) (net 23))
 (segment (start 118.745 50.165) (end 120.65 48.26) (width 0.5) (layer F.Cu) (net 24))
 (segment (start 118.745 52.07) (end 118.745 50.165) (width 0.5) (layer F.Cu) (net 24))
 (segment (start 115.57 55.245) (end 118.745 52.07) (width 0.5) (layer F.Cu) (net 24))
 (segment (start 113.03 55.245) (end 115.57 55.245) (width 0.5) (layer F.Cu) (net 24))
 (segment (start 113.03 53.275) (end 113.03 55.245) (width 0.5) (layer F.Cu) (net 24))
 (segment (start 121.92 61.595) (end 121.92 63.5) (width 0.5) (layer F.Cu) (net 5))
 (segment (start 121.285 60.96) (end 121.92 61.595) (width 0.5) (layer F.Cu) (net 5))
 (segment (start 120.015 60.96) (end 121.285 60.96) (width 0.5) (layer F.Cu) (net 5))
 (segment (start 118.84 59.785) (end 120.015 60.96) (width 0.5) (layer F.Cu) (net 5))
 (segment (start 118.84 58.42) (end 118.84 59.785) (width 0.5) (layer F.Cu) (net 5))
 (segment (start 118.84 57.245) (end 118.84 58.42) (width 0.5) (layer F.Cu) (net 5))
 (segment (start 118.11 56.515) (end 118.84 57.245) (width 0.5) (layer F.Cu) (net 5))
 (segment (start 112.395 56.515) (end 118.11 56.515) (width 0.5) (layer F.Cu) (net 5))
 (segment (start 111.76 55.88) (end 112.395 56.515) (width 0.5) (layer F.Cu) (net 5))
 (segment (start 111.76 53.275) (end 111.76 55.88) (width 0.5) (layer F.Cu) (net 5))
 (segment (start 119.38 64.77) (end 119.38 63.5) (width 0.5) (layer F.Cu) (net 4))
 (segment (start 120.015 65.405) (end 119.38 64.77) (width 0.5) (layer F.Cu) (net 4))
 (segment (start 123.19 65.405) (end 120.015 65.405) (width 0.5) (layer F.Cu) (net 4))
 (segment (start 123.5075 65.0875) (end 123.19 65.405) (width 0.5) (layer F.Cu) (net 4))
 (segment (start 113.03 48.325) (end 114.3 48.325) (width 0.5) (layer F.Cu) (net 4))
 (segment (start 98.425 46.15) (end 99.9 46.15) (width 0.5) (layer F.Cu) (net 4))
 (segment (start 99.9 46.15) (end 100.965 45.085) (width 0.5) (layer F.Cu) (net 4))
 (segment (start 100.965 45.085) (end 100.965 45.085) (width 0.5) (layer F.Cu) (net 4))
 (via (at 100.965 45.085) (size 1.5) (drill 0.5) (layers F.Cu B.Cu) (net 4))
 (segment (start 106.045 42.545) (end 106.045 42.545) (width 0.5) (layer F.Cu) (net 4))
 (via (at 106.045 42.545) (size 1.5) (drill 0.5) (layers F.Cu B.Cu) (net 4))
 (segment (start 123.46 58.4675) (end 123.5075 58.42) (width 0.5) (layer F.Cu) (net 4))
 (segment (start 121.285 58.4675) (end 123.46 58.4675) (width 0.5) (layer F.Cu) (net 4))
 (segment (start 123.5075 58.42) (end 123.5075 65.0875) (width 0.5) (layer F.Cu) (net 4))
 (segment (start 113.03 48.325) (end 113.03 42.545) (width 0.5) (layer F.Cu) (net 4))
 (segment (start 114.3 42.545) (end 106.045 42.545) (width 0.5) (layer F.Cu) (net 4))
 (segment (start 115.57 42.545) (end 114.3 42.545) (width 0.5) (layer F.Cu) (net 4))
 (segment (start 117.475 40.64) (end 115.57 42.545) (width 0.5) (layer F.Cu) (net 4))
 (segment (start 122.555 40.64) (end 117.475 40.64) (width 0.5) (layer F.Cu) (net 4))
 (segment (start 123.5075 41.5925) (end 122.555 40.64) (width 0.5) (layer F.Cu) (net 4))
 (segment (start 123.5075 58.42) (end 123.5075 41.5925) (width 0.5) (layer F.Cu) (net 4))
 (segment (start 103.505 42.545) (end 100.965 45.085) (width 0.5) (layer B.Cu) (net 4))
 (segment (start 106.045 42.545) (end 103.505 42.545) (width 0.5) (layer B.Cu) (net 4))
 (segment (start 111.76 64.77) (end 111.76 63.5) (width 0.5) (layer F.Cu) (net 1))
 (segment (start 111.125 65.405) (end 111.76 64.77) (width 0.5) (layer F.Cu) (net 1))
 (segment (start 87.63 65.405) (end 111.125 65.405) (width 0.5) (layer F.Cu) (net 1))
 (segment (start 86.995 64.77) (end 87.63 65.405) (width 0.5) (layer F.Cu) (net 1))
 (segment (start 86.995 55.45) (end 86.995 64.77) (width 0.5) (layer F.Cu) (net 1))
 (segment (start 110.49 48.325) (end 111.76 48.325) (width 0.5) (layer F.Cu) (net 25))
 (segment (start 97.155 46.15) (end 97.155 52.07) (width 0.5) (layer F.Cu) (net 26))
 (segment (start 97.155 52.07) (end 98.425 53.34) (width 0.5) (layer F.Cu) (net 26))
 (segment (start 98.425 53.34) (end 100.33 53.34) (width 0.5) (layer F.Cu) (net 26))
 (segment (start 100.33 53.34) (end 100.965 53.975) (width 0.5) (layer F.Cu) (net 26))
 (segment (start 100.965 53.975) (end 100.965 53.975) (width 0.5) (layer F.Cu) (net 26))
 (via (at 100.965 53.975) (size 1.5) (drill 0.5) (layers F.Cu B.Cu) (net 26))
 (via (at 104.14 53.975) (size 1.5) (drill 0.5) (layers F.Cu B.Cu) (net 26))
 (segment (start 104.84 53.275) (end 104.14 53.975) (width 0.5) (layer F.Cu) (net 26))
 (segment (start 106.68 53.275) (end 104.84 53.275) (width 0.5) (layer F.Cu) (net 26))
 (segment (start 100.965 53.975) (end 104.14 53.975) (width 0.5) (layer B.Cu) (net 26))
 (segment (start 107.95 53.275) (end 110.49 53.275) (width 0.5) (layer F.Cu) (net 27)))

